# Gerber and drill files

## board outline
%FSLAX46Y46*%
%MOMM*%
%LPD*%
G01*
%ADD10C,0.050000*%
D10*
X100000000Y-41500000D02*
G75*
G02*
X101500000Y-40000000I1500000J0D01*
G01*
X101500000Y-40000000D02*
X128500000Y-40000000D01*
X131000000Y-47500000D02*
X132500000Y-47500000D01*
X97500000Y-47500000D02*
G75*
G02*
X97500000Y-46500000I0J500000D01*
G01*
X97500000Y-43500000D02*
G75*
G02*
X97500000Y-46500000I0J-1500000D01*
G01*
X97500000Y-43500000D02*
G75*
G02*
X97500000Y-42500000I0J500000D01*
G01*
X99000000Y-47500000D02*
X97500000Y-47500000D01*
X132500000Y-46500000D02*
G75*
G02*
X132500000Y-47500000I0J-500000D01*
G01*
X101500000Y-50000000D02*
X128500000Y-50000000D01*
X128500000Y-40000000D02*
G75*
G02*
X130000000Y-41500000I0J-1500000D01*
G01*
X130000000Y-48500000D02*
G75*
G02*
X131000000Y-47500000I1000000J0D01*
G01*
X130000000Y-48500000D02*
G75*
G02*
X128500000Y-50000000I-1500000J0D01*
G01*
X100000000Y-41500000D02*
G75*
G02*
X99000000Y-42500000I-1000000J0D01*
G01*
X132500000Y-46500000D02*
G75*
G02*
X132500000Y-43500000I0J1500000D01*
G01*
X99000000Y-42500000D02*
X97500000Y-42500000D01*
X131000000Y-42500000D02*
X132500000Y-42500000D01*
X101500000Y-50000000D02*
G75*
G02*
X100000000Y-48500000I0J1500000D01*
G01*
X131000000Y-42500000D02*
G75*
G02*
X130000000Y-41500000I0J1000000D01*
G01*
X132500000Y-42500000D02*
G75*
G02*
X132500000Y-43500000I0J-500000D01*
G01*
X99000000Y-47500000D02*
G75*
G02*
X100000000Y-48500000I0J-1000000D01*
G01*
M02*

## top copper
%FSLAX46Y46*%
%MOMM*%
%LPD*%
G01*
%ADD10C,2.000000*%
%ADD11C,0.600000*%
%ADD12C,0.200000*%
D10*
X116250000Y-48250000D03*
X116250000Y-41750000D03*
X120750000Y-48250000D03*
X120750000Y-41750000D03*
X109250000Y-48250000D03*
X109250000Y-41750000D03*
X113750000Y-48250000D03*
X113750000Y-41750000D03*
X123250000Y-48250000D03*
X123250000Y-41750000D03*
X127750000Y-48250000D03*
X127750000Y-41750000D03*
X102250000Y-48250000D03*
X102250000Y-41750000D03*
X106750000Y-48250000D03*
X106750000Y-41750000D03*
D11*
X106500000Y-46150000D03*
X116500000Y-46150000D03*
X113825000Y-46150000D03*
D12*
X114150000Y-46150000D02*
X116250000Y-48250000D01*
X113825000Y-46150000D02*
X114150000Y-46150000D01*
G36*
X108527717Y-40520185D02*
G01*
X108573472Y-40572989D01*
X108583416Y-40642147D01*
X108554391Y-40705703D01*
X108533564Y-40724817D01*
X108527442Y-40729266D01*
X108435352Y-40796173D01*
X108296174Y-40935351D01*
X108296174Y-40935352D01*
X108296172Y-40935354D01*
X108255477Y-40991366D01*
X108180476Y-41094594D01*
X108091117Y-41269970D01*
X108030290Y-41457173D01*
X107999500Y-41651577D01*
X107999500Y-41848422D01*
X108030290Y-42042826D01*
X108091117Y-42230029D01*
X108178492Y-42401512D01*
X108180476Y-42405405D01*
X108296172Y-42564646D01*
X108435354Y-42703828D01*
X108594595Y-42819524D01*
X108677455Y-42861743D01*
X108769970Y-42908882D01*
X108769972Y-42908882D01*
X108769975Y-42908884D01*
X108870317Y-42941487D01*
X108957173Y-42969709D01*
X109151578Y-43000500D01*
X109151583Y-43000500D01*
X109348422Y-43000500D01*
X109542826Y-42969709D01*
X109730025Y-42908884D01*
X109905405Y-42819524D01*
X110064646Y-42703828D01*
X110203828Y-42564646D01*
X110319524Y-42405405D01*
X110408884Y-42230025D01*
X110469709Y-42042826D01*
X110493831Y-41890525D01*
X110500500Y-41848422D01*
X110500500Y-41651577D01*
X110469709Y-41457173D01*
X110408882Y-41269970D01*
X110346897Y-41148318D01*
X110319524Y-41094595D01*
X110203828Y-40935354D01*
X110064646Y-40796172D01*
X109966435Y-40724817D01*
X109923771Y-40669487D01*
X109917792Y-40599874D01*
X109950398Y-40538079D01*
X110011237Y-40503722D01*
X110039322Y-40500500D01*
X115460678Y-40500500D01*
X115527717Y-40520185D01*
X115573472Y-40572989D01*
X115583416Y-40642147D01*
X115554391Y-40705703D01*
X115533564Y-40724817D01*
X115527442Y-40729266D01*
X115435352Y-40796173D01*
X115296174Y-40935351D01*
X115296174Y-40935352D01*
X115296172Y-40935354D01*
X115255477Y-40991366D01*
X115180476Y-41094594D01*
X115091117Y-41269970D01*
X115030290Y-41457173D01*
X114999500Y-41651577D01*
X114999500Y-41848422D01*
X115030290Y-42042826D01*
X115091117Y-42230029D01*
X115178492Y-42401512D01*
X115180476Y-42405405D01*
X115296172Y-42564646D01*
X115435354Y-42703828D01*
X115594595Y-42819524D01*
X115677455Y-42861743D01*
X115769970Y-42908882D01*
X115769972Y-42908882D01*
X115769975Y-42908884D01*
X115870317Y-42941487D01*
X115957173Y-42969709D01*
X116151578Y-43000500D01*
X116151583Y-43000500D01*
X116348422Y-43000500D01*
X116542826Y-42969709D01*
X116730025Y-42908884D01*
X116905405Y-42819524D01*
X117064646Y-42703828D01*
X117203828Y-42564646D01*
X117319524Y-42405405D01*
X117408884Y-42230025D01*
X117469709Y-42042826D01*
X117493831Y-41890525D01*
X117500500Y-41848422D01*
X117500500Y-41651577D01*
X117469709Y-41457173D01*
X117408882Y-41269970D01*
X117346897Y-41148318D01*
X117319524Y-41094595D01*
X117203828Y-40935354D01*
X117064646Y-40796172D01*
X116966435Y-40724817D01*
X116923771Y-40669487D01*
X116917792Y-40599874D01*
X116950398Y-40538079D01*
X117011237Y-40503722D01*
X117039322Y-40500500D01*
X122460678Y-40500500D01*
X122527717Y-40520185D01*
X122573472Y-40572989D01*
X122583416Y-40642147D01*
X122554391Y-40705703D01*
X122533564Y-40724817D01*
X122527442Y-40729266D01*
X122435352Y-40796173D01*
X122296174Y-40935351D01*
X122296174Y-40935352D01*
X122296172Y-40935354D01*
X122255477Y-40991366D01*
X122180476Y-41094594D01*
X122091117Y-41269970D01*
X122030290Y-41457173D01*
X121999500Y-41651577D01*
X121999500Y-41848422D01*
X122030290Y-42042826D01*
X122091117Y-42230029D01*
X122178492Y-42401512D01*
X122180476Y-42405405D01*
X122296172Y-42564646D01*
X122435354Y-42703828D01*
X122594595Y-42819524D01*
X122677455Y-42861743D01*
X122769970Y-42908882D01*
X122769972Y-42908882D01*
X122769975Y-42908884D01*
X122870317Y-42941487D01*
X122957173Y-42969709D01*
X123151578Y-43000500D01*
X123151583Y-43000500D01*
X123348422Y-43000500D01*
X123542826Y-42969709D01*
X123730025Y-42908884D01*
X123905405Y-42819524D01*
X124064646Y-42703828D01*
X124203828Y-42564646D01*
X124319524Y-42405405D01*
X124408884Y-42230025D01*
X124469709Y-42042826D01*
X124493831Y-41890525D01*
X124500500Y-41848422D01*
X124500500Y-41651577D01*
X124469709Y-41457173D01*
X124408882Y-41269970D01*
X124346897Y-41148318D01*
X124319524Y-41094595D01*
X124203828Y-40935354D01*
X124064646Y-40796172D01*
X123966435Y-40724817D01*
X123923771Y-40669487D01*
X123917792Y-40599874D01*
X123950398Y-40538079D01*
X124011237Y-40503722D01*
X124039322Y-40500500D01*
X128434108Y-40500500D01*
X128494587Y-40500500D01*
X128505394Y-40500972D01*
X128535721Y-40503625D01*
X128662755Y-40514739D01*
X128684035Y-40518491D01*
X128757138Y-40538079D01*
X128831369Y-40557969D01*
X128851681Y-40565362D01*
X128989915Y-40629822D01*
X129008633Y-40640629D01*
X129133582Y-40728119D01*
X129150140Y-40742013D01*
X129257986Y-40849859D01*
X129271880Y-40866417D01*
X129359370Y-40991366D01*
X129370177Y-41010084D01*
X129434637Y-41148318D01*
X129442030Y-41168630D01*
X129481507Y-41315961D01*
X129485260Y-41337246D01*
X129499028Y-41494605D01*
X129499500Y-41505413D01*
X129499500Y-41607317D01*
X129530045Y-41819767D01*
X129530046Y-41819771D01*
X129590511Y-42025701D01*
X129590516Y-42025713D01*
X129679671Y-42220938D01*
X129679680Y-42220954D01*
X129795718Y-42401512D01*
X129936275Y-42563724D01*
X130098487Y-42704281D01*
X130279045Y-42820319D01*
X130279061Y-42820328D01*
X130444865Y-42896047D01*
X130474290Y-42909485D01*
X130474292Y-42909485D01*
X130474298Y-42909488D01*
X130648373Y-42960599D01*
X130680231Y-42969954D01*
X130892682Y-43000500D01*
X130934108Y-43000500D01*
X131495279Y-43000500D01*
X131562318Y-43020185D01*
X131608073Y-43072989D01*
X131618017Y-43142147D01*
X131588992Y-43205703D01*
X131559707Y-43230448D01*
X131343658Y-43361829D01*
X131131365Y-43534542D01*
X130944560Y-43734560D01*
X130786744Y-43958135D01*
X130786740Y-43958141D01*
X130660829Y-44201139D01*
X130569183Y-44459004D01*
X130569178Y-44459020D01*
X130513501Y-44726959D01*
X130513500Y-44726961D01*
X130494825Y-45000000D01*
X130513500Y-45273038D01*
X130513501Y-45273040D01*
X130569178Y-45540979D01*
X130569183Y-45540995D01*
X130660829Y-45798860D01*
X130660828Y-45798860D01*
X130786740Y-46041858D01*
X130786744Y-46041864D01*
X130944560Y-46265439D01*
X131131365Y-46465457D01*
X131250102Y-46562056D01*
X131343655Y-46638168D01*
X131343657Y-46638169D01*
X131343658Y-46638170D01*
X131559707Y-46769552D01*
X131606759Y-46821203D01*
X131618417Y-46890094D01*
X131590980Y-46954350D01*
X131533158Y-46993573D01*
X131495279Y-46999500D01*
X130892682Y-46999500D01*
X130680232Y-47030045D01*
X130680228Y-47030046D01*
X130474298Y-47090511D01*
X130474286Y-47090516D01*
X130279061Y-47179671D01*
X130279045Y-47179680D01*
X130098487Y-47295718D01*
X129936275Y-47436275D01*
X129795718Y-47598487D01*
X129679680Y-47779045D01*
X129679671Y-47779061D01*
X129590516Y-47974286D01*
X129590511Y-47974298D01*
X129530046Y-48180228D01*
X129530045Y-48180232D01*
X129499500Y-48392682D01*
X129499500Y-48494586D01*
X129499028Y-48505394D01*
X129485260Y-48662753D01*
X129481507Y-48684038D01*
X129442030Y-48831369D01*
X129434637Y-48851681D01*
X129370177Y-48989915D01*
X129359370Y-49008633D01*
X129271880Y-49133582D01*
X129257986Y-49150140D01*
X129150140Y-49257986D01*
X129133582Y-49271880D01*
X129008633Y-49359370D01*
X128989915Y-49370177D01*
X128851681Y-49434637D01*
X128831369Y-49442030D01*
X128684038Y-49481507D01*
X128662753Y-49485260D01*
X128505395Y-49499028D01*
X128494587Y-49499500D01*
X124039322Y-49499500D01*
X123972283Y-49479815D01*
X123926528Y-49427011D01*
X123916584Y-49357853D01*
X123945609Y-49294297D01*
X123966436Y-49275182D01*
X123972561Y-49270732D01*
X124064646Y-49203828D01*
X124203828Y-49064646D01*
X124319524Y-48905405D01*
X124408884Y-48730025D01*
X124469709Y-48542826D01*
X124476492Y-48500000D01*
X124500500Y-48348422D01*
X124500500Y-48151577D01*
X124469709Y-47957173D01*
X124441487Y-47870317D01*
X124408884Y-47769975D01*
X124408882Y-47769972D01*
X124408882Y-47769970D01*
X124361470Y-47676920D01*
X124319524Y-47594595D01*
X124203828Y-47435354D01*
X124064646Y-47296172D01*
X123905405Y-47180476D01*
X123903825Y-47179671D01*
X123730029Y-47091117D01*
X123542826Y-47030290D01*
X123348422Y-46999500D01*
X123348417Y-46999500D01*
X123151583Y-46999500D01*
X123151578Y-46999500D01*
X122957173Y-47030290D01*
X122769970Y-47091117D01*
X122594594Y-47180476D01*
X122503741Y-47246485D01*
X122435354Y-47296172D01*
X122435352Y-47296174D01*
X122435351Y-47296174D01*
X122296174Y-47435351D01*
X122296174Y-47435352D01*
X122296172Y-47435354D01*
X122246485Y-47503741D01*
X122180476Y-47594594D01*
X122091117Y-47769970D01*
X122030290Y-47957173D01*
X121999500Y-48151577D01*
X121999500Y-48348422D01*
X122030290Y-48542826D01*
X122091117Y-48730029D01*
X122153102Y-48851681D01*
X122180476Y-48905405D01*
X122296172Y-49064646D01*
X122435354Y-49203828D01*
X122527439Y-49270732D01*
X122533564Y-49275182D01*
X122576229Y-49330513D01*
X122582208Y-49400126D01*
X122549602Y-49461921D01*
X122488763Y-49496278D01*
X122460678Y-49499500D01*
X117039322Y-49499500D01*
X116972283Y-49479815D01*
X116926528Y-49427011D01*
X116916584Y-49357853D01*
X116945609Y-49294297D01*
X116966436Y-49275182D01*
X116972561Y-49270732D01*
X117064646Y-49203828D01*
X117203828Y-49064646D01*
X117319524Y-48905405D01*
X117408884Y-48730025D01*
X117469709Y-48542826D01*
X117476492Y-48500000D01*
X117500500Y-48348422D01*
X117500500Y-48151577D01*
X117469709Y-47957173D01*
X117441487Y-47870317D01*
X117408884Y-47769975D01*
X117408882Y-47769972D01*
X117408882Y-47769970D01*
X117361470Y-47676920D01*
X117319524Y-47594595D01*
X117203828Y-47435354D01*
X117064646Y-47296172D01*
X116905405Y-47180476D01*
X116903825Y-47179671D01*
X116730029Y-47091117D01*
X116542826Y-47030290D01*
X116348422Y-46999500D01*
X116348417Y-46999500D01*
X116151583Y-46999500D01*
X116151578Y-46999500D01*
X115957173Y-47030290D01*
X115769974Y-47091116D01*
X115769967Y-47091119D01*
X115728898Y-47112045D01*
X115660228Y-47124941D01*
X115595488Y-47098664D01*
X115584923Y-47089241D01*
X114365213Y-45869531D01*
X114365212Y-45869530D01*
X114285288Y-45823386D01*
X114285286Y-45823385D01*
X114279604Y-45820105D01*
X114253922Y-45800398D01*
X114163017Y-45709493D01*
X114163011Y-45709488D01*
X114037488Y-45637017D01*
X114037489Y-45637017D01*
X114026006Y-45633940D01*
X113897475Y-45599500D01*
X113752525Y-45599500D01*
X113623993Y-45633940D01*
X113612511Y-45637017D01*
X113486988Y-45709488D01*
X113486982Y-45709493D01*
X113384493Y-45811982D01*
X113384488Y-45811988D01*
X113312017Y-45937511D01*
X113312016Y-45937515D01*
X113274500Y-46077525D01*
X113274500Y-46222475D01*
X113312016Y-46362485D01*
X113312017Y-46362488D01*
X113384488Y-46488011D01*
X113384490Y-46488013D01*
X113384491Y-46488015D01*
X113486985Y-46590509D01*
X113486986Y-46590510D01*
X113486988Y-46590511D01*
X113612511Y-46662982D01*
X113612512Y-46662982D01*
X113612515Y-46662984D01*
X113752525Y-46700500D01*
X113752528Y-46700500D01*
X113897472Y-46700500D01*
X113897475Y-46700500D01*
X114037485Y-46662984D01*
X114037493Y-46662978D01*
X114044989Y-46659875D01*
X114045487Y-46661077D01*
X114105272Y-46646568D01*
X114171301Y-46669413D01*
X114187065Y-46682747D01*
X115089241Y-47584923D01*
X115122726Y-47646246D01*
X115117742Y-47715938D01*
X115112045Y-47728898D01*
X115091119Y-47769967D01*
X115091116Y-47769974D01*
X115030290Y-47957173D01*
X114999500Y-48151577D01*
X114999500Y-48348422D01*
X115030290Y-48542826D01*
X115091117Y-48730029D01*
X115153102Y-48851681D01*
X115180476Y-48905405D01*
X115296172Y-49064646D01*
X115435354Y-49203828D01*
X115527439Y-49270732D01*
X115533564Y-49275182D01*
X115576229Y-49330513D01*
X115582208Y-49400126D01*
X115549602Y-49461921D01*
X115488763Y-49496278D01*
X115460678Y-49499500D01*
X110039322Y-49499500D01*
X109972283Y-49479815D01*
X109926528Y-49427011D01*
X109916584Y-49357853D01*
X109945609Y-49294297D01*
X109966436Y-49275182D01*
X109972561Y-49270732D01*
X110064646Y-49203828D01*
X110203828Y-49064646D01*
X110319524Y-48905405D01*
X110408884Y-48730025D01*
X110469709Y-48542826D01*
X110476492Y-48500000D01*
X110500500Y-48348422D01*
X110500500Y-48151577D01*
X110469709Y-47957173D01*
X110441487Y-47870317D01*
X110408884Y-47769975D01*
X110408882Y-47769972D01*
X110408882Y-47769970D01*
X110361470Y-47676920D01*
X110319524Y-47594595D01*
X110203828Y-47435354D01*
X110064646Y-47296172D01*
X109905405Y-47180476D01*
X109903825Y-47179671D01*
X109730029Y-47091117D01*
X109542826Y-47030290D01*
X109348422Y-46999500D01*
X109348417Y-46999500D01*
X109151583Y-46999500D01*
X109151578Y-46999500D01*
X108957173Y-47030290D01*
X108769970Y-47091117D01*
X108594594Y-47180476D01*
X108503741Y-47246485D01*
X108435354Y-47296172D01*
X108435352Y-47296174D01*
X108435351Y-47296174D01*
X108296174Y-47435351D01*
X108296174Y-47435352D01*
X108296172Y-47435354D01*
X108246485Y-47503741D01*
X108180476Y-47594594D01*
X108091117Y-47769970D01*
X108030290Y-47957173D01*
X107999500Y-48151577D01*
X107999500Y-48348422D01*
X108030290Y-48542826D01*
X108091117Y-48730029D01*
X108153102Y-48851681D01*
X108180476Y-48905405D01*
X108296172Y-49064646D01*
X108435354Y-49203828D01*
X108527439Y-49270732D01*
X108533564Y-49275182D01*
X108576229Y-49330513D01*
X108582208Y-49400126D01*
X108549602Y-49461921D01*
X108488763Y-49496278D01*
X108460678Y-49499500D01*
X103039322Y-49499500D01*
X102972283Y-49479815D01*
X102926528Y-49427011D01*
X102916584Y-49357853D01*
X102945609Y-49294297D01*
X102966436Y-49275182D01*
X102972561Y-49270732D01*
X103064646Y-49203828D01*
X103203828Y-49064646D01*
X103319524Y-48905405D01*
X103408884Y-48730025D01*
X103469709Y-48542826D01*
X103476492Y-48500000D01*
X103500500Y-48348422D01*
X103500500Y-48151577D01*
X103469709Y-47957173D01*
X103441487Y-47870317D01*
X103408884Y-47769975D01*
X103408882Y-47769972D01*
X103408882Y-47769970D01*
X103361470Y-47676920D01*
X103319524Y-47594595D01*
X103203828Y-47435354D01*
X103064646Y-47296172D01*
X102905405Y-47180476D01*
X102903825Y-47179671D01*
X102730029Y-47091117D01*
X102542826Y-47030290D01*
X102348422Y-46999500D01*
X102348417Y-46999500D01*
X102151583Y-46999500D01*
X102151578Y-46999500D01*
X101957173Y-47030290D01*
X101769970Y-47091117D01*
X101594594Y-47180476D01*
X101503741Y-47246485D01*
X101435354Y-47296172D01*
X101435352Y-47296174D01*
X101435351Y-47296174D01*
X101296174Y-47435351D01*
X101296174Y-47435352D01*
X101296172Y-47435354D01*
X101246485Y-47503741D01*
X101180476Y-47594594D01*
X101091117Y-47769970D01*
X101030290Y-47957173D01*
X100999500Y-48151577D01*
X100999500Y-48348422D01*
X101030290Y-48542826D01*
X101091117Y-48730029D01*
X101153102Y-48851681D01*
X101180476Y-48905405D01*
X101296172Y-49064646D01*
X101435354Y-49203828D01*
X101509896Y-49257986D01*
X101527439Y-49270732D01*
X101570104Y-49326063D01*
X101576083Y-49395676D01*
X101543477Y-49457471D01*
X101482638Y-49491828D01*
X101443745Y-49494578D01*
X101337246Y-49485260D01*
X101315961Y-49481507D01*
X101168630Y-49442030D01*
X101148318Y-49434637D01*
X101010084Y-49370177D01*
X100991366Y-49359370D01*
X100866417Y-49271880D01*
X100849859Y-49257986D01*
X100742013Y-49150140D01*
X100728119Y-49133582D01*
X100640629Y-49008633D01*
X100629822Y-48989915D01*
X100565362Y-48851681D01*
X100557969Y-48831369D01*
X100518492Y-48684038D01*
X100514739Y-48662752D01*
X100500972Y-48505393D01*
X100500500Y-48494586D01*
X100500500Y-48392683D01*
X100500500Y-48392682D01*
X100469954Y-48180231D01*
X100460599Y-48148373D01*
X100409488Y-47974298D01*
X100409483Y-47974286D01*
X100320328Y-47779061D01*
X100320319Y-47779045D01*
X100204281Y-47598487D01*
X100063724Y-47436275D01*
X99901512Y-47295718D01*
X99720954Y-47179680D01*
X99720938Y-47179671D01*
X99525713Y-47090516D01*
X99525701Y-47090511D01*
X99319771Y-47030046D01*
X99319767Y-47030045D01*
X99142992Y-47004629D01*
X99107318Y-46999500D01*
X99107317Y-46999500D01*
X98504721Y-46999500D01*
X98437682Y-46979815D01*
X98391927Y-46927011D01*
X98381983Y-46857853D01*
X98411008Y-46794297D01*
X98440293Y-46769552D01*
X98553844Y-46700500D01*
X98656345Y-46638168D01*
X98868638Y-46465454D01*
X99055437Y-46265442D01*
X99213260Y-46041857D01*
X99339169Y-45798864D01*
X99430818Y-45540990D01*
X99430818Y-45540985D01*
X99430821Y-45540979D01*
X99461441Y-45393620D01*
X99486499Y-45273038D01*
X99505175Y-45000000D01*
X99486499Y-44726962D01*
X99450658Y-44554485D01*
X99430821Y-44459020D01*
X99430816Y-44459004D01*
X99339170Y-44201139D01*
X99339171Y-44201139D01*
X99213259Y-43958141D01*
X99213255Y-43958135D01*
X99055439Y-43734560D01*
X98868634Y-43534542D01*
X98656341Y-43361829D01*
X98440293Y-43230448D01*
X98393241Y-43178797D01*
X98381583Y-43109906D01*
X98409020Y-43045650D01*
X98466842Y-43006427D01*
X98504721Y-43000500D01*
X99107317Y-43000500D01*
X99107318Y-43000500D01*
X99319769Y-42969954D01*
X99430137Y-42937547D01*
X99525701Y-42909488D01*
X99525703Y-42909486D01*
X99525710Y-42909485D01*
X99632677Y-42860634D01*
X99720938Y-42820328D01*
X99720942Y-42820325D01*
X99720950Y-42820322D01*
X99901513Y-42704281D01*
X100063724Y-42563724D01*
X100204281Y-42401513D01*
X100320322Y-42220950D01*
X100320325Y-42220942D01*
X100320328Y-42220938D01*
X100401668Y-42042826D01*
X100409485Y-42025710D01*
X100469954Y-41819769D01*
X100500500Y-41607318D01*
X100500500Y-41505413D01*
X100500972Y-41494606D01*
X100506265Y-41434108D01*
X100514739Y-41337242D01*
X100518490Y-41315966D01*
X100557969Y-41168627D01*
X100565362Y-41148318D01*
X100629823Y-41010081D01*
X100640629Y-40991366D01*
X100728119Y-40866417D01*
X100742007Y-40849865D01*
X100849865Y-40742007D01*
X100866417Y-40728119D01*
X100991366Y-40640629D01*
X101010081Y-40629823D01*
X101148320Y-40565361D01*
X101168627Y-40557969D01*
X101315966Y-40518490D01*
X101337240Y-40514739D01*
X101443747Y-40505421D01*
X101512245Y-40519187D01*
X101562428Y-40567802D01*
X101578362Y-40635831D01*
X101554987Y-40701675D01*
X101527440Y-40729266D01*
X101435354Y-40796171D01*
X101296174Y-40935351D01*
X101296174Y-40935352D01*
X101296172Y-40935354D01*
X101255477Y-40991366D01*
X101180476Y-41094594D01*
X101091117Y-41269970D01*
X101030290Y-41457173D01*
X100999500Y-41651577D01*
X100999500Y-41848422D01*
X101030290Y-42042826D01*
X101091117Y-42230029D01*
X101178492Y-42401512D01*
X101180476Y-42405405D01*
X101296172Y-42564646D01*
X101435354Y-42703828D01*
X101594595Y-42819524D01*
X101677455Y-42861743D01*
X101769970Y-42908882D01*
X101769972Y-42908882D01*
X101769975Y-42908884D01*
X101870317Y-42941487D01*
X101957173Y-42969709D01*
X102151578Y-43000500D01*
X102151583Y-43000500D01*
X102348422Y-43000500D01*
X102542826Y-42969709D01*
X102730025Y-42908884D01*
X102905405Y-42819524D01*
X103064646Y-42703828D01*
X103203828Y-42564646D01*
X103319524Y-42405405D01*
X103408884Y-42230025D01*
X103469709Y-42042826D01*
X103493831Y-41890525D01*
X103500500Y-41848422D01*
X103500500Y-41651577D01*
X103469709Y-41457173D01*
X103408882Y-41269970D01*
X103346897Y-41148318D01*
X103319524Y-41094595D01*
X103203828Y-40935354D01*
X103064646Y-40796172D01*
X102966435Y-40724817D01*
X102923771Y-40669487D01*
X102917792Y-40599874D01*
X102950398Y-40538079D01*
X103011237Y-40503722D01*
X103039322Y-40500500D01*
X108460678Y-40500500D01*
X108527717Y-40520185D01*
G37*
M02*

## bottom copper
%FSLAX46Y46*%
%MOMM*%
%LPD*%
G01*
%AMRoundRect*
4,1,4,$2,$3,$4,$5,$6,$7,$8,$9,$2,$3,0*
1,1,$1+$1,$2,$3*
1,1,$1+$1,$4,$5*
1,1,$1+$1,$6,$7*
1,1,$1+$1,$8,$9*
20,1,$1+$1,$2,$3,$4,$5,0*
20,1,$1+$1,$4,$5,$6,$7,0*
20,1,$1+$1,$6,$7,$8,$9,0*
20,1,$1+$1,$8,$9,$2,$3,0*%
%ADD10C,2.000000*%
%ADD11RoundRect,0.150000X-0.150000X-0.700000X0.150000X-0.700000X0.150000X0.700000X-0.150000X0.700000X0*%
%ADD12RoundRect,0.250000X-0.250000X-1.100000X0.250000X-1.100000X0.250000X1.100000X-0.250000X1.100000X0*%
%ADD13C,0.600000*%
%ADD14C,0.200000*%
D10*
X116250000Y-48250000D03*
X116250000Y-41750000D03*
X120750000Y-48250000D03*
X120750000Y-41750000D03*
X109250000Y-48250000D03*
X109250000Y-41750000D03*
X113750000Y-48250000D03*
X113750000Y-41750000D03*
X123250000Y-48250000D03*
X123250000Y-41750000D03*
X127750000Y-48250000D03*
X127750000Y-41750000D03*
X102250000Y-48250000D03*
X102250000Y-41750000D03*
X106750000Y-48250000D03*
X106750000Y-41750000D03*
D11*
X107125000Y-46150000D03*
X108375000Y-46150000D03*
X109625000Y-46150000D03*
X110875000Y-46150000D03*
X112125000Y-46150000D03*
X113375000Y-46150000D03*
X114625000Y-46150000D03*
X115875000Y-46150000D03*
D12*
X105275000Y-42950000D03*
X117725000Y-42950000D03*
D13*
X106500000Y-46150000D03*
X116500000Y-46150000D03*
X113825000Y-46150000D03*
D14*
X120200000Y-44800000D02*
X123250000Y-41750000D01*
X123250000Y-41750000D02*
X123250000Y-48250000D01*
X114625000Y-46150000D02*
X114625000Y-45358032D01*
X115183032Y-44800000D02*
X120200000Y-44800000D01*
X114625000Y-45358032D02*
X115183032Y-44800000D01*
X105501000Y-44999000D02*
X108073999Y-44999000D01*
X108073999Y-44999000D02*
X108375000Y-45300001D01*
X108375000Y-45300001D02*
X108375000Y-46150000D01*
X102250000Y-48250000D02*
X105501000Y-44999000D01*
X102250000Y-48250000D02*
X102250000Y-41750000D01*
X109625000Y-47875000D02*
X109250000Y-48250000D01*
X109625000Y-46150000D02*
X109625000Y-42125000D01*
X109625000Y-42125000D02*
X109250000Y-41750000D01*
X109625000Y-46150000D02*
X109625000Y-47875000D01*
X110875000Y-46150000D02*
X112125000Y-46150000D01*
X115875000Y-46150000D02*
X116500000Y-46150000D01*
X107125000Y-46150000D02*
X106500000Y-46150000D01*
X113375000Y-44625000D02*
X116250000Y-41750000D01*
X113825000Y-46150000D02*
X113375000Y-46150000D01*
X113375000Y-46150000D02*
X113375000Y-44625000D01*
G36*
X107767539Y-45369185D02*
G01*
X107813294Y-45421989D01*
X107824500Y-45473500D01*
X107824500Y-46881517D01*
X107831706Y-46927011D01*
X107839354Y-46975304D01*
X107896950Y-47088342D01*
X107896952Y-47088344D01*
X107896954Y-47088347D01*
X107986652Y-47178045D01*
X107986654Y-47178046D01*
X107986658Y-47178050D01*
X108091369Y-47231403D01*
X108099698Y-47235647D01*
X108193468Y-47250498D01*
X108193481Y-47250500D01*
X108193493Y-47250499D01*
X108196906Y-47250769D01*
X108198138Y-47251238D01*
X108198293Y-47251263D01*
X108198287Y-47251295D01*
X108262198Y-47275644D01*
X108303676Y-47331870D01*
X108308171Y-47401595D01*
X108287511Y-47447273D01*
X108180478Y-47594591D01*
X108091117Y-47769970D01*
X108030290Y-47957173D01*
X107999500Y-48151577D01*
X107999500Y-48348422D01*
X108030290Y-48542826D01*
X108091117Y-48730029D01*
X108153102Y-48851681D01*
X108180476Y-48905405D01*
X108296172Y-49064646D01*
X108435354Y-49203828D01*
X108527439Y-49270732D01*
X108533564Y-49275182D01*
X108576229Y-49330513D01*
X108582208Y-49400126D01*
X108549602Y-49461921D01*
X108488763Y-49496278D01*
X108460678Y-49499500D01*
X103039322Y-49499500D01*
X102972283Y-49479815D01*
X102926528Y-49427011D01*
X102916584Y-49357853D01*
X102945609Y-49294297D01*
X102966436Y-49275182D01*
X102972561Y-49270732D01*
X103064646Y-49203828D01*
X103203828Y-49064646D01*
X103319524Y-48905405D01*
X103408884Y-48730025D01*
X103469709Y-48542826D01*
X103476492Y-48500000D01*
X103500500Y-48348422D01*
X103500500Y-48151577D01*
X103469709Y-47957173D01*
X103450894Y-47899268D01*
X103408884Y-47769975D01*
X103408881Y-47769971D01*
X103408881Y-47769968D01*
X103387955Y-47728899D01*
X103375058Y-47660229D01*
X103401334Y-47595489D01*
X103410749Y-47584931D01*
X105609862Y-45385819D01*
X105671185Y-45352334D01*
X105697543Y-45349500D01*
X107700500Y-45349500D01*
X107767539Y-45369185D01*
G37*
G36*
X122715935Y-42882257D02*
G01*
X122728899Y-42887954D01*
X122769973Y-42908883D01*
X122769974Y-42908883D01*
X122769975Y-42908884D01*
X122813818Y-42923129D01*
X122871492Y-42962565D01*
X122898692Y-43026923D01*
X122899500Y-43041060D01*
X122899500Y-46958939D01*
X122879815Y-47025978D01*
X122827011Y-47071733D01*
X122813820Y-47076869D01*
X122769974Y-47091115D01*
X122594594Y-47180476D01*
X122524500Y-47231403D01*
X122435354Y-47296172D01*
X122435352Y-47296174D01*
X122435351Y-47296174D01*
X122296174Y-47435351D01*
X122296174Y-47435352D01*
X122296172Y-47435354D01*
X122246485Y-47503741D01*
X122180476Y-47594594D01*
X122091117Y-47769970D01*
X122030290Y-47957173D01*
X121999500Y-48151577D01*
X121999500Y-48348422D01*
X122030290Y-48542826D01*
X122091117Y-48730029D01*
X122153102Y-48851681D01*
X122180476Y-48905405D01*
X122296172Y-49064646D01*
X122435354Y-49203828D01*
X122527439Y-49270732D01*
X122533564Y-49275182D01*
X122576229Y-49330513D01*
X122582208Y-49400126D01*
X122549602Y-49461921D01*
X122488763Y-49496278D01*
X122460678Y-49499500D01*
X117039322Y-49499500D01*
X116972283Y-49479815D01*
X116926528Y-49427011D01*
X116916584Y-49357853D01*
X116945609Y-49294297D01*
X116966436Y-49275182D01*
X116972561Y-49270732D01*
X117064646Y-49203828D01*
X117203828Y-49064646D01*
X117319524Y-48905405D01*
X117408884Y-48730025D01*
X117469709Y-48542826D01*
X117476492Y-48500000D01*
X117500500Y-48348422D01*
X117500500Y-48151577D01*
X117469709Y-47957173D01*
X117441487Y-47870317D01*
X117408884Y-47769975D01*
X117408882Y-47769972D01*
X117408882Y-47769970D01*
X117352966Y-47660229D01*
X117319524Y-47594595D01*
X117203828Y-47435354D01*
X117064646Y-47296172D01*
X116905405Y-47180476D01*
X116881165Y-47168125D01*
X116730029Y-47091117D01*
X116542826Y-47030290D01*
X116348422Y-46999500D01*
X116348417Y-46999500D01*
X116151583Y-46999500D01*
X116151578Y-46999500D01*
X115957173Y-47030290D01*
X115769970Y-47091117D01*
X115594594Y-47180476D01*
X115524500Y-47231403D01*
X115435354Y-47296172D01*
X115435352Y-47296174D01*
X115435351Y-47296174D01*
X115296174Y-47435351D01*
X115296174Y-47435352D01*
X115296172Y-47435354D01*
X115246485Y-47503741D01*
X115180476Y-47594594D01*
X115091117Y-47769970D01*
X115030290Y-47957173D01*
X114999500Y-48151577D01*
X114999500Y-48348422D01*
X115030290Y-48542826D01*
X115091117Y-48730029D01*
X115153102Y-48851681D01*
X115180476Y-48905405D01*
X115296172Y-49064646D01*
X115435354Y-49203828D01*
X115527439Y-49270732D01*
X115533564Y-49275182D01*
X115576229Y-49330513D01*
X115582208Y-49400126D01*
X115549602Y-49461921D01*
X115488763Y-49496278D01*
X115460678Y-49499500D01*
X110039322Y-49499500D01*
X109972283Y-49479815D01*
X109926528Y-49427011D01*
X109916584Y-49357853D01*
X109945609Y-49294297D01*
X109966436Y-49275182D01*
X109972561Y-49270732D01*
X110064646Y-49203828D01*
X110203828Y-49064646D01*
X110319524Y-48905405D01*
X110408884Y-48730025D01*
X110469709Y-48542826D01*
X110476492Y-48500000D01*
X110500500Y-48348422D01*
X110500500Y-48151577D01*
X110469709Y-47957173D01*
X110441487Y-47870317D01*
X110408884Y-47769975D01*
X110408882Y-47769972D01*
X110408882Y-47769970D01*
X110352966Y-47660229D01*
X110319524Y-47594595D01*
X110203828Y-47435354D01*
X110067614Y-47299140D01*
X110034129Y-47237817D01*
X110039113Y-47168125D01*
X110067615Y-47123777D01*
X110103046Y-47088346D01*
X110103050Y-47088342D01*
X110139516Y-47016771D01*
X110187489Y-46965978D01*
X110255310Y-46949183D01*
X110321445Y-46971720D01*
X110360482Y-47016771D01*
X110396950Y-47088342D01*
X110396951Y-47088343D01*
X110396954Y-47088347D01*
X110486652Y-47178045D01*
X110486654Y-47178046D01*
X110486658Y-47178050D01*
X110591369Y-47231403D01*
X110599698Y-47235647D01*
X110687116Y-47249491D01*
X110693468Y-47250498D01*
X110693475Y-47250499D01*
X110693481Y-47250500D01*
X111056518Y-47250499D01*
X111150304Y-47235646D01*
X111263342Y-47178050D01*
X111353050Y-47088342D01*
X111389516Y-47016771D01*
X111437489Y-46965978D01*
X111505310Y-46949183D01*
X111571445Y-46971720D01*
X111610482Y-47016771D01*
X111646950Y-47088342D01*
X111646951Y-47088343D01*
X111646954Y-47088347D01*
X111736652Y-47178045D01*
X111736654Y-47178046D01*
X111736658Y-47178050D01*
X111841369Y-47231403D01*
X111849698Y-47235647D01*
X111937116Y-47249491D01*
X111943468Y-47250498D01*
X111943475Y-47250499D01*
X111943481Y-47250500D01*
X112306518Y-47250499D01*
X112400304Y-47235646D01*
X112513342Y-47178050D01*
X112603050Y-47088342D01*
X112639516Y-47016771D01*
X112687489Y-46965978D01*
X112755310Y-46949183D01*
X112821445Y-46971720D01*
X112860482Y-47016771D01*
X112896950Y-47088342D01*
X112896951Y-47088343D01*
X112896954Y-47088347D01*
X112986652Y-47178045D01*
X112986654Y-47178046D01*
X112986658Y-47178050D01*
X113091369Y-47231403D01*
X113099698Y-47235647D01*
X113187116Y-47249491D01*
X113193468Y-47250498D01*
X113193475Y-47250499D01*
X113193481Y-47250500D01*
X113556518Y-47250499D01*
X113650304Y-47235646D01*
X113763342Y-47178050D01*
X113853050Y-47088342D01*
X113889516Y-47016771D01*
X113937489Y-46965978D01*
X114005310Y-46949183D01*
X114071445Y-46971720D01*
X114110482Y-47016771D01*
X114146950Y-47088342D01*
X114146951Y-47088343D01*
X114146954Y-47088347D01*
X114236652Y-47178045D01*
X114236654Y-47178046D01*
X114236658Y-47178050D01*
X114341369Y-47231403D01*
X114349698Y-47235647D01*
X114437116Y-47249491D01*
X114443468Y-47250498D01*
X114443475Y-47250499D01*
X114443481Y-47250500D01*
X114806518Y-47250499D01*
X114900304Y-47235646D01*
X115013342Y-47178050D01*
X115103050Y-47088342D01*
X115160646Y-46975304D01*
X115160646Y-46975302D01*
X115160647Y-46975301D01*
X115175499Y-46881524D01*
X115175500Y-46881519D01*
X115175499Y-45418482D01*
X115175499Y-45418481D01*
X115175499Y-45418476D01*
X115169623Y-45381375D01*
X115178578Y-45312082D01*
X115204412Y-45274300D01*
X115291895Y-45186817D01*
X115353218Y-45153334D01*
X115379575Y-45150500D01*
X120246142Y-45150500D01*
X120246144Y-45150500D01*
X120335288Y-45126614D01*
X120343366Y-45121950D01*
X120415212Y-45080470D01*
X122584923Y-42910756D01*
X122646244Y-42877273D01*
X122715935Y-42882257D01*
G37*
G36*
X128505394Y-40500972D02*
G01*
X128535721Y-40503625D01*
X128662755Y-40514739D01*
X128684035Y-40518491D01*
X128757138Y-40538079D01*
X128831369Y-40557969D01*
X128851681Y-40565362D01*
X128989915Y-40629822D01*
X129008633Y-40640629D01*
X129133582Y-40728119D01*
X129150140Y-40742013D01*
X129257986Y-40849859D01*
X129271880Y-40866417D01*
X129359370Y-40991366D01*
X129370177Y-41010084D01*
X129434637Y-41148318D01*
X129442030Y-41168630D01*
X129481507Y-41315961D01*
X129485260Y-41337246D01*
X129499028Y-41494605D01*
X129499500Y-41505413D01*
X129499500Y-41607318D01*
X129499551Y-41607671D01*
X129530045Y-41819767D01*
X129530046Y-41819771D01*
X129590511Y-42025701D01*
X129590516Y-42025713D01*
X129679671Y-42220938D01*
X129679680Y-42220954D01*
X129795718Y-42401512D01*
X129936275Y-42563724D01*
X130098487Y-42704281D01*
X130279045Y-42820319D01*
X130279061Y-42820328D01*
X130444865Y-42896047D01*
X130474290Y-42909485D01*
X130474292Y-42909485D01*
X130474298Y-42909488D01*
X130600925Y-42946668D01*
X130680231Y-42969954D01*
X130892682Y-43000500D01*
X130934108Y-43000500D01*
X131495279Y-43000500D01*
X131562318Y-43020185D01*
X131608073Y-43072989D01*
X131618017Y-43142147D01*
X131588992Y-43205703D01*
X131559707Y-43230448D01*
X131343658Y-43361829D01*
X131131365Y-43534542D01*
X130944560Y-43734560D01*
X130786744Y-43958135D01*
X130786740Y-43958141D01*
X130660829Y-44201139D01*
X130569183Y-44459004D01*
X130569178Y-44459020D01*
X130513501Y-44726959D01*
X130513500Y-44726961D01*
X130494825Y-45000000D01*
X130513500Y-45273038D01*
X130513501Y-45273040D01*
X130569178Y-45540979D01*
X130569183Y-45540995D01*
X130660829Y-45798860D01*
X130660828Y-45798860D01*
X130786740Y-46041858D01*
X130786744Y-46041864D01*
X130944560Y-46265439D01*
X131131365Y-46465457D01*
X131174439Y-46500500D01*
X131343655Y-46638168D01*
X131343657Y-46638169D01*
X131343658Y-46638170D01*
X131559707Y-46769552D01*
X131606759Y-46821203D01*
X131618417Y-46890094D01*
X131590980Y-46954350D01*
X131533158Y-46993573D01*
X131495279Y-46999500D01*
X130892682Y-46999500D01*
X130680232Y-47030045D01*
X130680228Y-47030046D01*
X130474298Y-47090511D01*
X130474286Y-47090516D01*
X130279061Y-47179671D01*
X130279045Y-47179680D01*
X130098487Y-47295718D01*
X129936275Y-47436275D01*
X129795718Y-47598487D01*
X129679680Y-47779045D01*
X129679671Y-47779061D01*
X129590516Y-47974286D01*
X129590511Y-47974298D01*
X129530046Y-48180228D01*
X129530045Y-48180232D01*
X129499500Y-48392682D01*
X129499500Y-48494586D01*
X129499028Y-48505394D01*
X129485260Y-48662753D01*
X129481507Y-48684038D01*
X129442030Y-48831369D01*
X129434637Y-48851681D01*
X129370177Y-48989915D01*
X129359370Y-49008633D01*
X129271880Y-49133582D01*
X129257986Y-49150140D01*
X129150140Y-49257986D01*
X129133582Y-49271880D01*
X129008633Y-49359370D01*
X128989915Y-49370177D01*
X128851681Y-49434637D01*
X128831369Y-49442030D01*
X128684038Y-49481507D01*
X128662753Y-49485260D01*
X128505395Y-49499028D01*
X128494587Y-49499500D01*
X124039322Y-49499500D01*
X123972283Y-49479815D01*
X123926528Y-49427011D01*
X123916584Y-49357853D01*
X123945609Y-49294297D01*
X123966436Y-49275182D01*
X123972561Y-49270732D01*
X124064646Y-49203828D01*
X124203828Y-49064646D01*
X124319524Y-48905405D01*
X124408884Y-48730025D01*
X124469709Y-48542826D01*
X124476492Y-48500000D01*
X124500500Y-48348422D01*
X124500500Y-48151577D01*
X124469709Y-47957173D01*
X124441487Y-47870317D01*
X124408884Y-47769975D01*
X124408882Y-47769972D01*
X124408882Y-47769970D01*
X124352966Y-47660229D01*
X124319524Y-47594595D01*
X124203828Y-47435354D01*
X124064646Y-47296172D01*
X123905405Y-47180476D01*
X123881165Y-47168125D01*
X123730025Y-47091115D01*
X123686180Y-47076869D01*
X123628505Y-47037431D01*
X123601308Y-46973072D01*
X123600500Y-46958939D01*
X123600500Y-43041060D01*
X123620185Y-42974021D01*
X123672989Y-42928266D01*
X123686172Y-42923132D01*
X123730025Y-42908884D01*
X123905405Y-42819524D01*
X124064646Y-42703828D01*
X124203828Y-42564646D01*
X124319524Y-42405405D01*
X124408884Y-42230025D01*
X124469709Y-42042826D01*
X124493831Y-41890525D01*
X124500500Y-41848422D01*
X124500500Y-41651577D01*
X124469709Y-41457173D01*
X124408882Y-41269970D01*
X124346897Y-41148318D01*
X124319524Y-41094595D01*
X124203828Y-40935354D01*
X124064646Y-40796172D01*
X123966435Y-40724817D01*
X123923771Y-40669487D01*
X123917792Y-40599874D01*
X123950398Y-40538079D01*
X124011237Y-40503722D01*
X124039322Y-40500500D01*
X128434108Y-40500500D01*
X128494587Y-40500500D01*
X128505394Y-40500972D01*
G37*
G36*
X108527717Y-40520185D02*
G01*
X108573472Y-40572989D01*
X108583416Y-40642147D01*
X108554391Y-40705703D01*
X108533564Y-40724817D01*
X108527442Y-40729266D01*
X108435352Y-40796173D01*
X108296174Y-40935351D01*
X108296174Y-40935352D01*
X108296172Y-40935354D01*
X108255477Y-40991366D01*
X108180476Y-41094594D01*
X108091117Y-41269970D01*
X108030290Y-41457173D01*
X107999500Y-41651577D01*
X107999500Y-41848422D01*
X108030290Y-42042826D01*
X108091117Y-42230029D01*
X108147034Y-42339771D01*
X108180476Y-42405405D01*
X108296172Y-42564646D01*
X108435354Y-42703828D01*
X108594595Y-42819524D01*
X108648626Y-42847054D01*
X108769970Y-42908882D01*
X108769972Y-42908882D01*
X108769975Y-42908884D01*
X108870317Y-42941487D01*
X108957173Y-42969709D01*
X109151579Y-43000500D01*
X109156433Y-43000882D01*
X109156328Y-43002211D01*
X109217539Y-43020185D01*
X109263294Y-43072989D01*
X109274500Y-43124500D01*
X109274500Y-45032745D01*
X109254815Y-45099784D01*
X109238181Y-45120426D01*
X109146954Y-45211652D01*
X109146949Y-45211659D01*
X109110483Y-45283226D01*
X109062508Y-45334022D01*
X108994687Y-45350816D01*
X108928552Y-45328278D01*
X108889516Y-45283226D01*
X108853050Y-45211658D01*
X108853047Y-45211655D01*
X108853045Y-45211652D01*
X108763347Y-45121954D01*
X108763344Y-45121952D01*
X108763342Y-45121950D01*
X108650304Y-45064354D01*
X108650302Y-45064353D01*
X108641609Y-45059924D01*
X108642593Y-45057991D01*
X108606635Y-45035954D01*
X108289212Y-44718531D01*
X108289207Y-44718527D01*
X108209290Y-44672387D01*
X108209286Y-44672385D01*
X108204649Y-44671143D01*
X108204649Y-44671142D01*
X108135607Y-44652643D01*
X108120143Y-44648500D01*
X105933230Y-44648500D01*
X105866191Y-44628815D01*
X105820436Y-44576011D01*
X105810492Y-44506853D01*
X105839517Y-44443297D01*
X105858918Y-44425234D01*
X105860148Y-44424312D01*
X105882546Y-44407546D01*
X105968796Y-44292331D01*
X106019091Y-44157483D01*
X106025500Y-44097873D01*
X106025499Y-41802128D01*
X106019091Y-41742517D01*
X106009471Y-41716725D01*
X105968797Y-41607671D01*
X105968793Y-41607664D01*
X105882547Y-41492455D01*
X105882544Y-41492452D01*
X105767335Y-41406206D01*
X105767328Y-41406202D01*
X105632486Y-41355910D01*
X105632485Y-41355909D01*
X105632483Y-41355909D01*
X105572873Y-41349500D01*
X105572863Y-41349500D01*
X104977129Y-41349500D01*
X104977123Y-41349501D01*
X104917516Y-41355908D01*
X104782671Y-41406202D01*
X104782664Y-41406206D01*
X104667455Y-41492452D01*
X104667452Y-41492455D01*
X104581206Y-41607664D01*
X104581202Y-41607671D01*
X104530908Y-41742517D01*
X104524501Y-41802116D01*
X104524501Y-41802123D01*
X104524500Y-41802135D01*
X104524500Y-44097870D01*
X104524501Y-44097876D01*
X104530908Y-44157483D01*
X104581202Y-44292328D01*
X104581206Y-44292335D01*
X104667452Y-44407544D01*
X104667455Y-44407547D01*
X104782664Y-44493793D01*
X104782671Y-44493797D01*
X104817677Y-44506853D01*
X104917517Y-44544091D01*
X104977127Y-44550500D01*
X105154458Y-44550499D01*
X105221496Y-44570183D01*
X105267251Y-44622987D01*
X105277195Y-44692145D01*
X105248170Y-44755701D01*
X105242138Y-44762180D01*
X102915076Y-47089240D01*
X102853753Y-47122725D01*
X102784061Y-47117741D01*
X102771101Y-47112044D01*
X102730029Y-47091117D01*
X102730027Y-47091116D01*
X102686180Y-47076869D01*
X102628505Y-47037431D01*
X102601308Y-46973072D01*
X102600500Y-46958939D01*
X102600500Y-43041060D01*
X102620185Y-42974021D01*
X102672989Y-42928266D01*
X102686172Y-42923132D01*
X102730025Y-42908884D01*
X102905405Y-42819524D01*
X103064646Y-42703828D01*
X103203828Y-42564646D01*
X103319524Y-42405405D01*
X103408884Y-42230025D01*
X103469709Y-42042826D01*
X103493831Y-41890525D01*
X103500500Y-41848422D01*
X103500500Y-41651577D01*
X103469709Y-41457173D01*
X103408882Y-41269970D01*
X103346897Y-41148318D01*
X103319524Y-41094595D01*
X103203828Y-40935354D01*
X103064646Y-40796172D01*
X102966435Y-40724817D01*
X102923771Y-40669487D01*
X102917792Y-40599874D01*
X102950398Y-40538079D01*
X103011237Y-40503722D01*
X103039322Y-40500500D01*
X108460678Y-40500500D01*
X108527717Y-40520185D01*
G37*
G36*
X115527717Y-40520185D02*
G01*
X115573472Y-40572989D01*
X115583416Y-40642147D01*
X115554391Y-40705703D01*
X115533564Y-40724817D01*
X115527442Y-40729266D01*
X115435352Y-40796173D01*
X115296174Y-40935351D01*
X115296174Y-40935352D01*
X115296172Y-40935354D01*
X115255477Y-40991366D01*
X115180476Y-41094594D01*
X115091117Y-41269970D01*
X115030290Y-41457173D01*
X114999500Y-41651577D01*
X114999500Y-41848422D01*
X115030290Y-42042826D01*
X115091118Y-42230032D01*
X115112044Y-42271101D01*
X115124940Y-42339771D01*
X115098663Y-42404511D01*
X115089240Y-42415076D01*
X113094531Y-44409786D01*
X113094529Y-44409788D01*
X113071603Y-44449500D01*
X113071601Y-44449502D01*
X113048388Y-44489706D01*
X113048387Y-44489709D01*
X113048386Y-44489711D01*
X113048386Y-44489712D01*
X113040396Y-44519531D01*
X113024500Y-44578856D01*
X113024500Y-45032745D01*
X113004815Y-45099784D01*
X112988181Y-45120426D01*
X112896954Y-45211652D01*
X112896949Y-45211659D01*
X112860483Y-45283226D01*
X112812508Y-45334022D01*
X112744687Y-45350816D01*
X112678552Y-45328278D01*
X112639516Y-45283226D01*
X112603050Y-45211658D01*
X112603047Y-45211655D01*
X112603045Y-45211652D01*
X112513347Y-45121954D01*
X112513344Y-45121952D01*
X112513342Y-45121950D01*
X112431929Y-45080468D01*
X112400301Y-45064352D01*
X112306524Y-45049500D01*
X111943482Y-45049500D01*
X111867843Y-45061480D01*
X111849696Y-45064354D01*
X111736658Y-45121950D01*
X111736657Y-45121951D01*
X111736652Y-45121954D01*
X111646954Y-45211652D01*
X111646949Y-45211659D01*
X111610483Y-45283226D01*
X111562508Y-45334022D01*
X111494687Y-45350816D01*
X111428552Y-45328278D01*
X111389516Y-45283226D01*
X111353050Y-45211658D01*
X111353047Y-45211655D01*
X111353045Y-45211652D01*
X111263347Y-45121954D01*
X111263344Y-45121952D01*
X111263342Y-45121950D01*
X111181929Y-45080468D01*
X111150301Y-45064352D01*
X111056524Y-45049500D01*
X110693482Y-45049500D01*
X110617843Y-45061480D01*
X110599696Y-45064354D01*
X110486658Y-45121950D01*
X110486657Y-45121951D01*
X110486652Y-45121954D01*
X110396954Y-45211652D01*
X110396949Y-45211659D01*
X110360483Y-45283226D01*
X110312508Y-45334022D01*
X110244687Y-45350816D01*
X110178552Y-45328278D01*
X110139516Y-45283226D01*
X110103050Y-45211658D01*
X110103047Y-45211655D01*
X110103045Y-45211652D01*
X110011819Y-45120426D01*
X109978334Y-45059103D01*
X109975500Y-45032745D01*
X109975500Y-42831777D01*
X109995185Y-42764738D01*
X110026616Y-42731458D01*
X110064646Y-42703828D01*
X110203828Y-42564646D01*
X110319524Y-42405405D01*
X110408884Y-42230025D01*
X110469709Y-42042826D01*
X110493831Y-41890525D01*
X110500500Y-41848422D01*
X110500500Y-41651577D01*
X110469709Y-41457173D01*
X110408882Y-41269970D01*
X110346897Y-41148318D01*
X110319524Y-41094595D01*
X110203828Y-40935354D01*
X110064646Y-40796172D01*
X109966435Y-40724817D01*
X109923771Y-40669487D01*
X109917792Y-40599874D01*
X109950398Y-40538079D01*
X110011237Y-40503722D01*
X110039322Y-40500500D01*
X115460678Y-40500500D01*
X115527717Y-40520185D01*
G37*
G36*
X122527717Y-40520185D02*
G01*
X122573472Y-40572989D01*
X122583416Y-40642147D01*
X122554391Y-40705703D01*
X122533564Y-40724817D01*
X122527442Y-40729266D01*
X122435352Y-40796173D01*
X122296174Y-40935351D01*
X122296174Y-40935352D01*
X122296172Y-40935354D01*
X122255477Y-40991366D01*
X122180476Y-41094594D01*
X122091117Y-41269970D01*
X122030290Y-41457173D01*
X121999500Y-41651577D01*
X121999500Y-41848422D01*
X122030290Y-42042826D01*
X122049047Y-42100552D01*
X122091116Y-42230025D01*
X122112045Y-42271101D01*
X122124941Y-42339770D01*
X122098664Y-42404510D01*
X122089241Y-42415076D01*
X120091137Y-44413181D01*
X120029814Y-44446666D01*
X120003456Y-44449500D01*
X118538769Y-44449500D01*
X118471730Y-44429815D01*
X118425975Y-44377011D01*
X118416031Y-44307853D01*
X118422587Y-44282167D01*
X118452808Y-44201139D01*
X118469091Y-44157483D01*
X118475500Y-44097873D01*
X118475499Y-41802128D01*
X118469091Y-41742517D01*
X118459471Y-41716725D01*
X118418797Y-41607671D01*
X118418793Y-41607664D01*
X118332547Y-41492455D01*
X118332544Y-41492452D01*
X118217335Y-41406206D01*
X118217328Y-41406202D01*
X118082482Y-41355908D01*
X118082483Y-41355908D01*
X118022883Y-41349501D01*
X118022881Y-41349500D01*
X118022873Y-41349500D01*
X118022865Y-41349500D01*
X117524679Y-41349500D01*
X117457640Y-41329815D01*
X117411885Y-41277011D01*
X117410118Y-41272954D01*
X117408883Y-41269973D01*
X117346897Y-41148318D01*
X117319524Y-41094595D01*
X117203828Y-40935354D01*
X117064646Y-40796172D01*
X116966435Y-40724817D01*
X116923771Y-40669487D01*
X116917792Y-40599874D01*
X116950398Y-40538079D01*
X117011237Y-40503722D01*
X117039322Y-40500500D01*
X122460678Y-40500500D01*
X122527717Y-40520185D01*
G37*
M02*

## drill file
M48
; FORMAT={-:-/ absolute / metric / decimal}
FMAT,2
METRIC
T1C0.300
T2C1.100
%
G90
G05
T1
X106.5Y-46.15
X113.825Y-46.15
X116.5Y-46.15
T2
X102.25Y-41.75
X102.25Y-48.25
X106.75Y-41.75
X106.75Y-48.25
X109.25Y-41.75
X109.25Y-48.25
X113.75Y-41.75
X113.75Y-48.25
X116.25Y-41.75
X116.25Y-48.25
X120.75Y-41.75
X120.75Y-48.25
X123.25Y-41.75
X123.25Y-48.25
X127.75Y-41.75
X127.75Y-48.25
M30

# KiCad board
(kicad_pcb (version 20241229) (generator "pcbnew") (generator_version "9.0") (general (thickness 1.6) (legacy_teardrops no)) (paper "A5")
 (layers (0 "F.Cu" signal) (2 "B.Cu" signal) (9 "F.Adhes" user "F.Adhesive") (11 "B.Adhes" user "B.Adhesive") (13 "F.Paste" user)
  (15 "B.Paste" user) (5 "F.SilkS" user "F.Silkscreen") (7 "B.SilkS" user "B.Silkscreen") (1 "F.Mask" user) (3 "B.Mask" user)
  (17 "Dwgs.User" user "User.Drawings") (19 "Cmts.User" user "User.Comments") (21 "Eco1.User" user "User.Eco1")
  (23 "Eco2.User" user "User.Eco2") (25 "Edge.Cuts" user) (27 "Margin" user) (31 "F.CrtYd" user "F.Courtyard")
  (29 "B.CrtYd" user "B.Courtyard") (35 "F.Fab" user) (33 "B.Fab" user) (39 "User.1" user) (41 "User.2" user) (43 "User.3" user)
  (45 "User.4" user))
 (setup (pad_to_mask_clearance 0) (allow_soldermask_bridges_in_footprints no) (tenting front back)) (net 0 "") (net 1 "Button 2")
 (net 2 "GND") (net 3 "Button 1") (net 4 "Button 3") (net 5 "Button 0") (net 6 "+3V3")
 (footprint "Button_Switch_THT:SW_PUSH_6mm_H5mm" (layer "F.Cu") (at 116.25 48.25 90)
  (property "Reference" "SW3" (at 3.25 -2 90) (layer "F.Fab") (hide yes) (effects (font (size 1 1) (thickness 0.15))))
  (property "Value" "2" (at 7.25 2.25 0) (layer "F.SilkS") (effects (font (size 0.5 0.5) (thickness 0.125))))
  (pad "1" thru_hole circle (at 0 0 180) (size 2 2) (drill 1.1) (layers "*.Cu" "*.Mask") (remove_unused_layers no) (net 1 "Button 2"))
  (pad "1" thru_hole circle (at 6.5 0 180) (size 2 2) (drill 1.1) (layers "*.Cu" "*.Mask") (remove_unused_layers no) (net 1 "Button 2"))
  (pad "2" thru_hole circle (at 0 4.5 180) (size 2 2) (drill 1.1) (layers "*.Cu" "*.Mask") (remove_unused_layers no) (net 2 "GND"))
  (pad "2" thru_hole circle (at 6.5 4.5 180) (size 2 2) (drill 1.1) (layers "*.Cu" "*.Mask") (remove_unused_layers no) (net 2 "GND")))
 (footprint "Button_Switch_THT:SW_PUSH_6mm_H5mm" (layer "F.Cu") (at 109.25 48.25 90)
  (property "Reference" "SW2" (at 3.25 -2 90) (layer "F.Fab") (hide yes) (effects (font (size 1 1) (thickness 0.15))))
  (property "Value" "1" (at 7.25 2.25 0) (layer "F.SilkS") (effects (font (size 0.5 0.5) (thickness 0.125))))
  (pad "1" thru_hole circle (at 0 0 180) (size 2 2) (drill 1.1) (layers "*.Cu" "*.Mask") (remove_unused_layers no) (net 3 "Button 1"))
  (pad "1" thru_hole circle (at 6.5 0 180) (size 2 2) (drill 1.1) (layers "*.Cu" "*.Mask") (remove_unused_layers no) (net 3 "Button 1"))
  (pad "2" thru_hole circle (at 0 4.5 180) (size 2 2) (drill 1.1) (layers "*.Cu" "*.Mask") (remove_unused_layers no) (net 2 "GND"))
  (pad "2" thru_hole circle (at 6.5 4.5 180) (size 2 2) (drill 1.1) (layers "*.Cu" "*.Mask") (remove_unused_layers no) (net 2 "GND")))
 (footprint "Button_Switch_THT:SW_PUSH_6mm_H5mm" (layer "F.Cu") (at 123.25 48.25 90)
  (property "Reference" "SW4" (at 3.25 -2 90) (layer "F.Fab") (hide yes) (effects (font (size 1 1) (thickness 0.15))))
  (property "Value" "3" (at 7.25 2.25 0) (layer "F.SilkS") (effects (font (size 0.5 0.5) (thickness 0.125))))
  (pad "1" thru_hole circle (at 0 0 180) (size 2 2) (drill 1.1) (layers "*.Cu" "*.Mask") (remove_unused_layers no) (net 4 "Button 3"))
  (pad "1" thru_hole circle (at 6.5 0 180) (size 2 2) (drill 1.1) (layers "*.Cu" "*.Mask") (remove_unused_layers no) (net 4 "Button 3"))
  (pad "2" thru_hole circle (at 0 4.5 180) (size 2 2) (drill 1.1) (layers "*.Cu" "*.Mask") (remove_unused_layers no) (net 2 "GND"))
  (pad "2" thru_hole circle (at 6.5 4.5 180) (size 2 2) (drill 1.1) (layers "*.Cu" "*.Mask") (remove_unused_layers no) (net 2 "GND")))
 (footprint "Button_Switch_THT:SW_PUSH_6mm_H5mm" (layer "F.Cu") (at 102.25 48.25 90)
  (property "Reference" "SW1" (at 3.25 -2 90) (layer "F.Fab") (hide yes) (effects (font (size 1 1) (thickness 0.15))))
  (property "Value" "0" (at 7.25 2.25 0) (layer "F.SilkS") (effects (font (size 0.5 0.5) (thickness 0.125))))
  (pad "1" thru_hole circle (at 0 0 180) (size 2 2) (drill 1.1) (layers "*.Cu" "*.Mask") (remove_unused_layers no) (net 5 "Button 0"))
  (pad "1" thru_hole circle (at 6.5 0 180) (size 2 2) (drill 1.1) (layers "*.Cu" "*.Mask") (remove_unused_layers no) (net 5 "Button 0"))
  (pad "2" thru_hole circle (at 0 4.5 180) (size 2 2) (drill 1.1) (layers "*.Cu" "*.Mask") (remove_unused_layers no) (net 2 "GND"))
  (pad "2" thru_hole circle (at 6.5 4.5 180) (size 2 2) (drill 1.1) (layers "*.Cu" "*.Mask") (remove_unused_layers no) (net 2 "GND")))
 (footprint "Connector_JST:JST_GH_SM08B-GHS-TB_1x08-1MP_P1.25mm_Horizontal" (layer "B.Cu") (at 111.5 44.3)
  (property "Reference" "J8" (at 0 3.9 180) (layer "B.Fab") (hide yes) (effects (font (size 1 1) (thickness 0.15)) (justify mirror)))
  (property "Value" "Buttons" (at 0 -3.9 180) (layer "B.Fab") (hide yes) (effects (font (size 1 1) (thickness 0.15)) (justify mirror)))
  (pad "1" smd roundrect (at -4.375 1.85) (size 0.6 1.7) (layers "B.Cu" "B.Mask" "B.Paste") (roundrect_rratio 0.25) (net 2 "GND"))
  (pad "2" smd roundrect (at -3.125 1.85) (size 0.6 1.7) (layers "B.Cu" "B.Mask" "B.Paste") (roundrect_rratio 0.25) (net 5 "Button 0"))
  (pad "3" smd roundrect (at -1.875 1.85) (size 0.6 1.7) (layers "B.Cu" "B.Mask" "B.Paste") (roundrect_rratio 0.25) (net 3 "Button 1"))
  (pad "4" smd roundrect (at -0.625 1.85) (size 0.6 1.7) (layers "B.Cu" "B.Mask" "B.Paste") (roundrect_rratio 0.25) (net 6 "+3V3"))
  (pad "5" smd roundrect (at 0.625 1.85) (size 0.6 1.7) (layers "B.Cu" "B.Mask" "B.Paste") (roundrect_rratio 0.25) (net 6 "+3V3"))
  (pad "6" smd roundrect (at 1.875 1.85) (size 0.6 1.7) (layers "B.Cu" "B.Mask" "B.Paste") (roundrect_rratio 0.25) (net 1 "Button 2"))
  (pad "7" smd roundrect (at 3.125 1.85) (size 0.6 1.7) (layers "B.Cu" "B.Mask" "B.Paste") (roundrect_rratio 0.25) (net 4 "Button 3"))
  (pad "8" smd roundrect (at 4.375 1.85) (size 0.6 1.7) (layers "B.Cu" "B.Mask" "B.Paste") (roundrect_rratio 0.25) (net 2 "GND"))
  (pad "MP" smd roundrect (at -6.225 -1.35) (size 1 2.7) (layers "B.Cu" "B.Mask" "B.Paste") (roundrect_rratio 0.25))
  (pad "MP" smd roundrect (at 6.225 -1.35) (size 1 2.7) (layers "B.Cu" "B.Mask" "B.Paste") (roundrect_rratio 0.25)))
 (gr_arc (start 100 41.5) (mid 100.43934 40.43934) (end 101.5 40) (stroke (width 0.05) (type default)) (layer "Edge.Cuts"))
 (gr_line (start 101.5 40) (end 128.5 40) (stroke (width 0.05) (type default)) (layer "Edge.Cuts"))
 (gr_line (start 131 47.5) (end 132.5 47.5) (stroke (width 0.05) (type default)) (layer "Edge.Cuts"))
 (gr_arc (start 97.5 47.5) (mid 97 47) (end 97.5 46.5) (stroke (width 0.05) (type default)) (layer "Edge.Cuts"))
 (gr_arc (start 97.5 43.5) (mid 99 45) (end 97.5 46.5) (stroke (width 0.05) (type default)) (layer "Edge.Cuts"))
 (gr_arc (start 97.5 43.5) (mid 97 43) (end 97.5 42.5) (stroke (width 0.05) (type default)) (layer "Edge.Cuts"))
 (gr_line (start 99 47.5) (end 97.5 47.5) (stroke (width 0.05) (type default)) (layer "Edge.Cuts"))
 (gr_arc (start 132.5 46.5) (mid 133 47) (end 132.5 47.5) (stroke (width 0.05) (type default)) (layer "Edge.Cuts"))
 (gr_line (start 101.5 50) (end 128.5 50) (stroke (width 0.05) (type default)) (layer "Edge.Cuts"))
 (gr_arc (start 128.5 40) (mid 129.56066 40.43934) (end 130 41.5) (stroke (width 0.05) (type default)) (layer "Edge.Cuts"))
 (gr_arc (start 130 48.5) (mid 130.292893 47.792893) (end 131 47.5) (stroke (width 0.05) (type default)) (layer "Edge.Cuts"))
 (gr_arc (start 130 48.5) (mid 129.56066 49.56066) (end 128.5 50) (stroke (width 0.05) (type default)) (layer "Edge.Cuts"))
 (gr_arc (start 100 41.5) (mid 99.707107 42.207107) (end 99 42.5) (stroke (width 0.05) (type default)) (layer "Edge.Cuts"))
 (gr_arc (start 132.5 46.5) (mid 131 45) (end 132.5 43.5) (stroke (width 0.05) (type default)) (layer "Edge.Cuts"))
 (gr_line (start 99 42.5) (end 97.5 42.5) (stroke (width 0.05) (type default)) (layer "Edge.Cuts"))
 (gr_line (start 131 42.5) (end 132.5 42.5) (stroke (width 0.05) (type default)) (layer "Edge.Cuts"))
 (gr_arc (start 101.5 50) (mid 100.43934 49.56066) (end 100 48.5) (stroke (width 0.05) (type default)) (layer "Edge.Cuts"))
 (gr_arc (start 131 42.5) (mid 130.292893 42.207107) (end 130 41.5) (stroke (width 0.05) (type default)) (layer "Edge.Cuts"))
 (gr_arc (start 132.5 42.5) (mid 133 43) (end 132.5 43.5) (stroke (width 0.05) (type default)) (layer "Edge.Cuts"))
 (gr_arc (start 99 47.5) (mid 99.707107 47.792893) (end 100 48.5) (stroke (width 0.05) (type default)) (layer "Edge.Cuts"))
 (segment (start 120.2 44.8) (end 123.25 41.75) (width 0.2) (layer "B.Cu") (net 4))
 (segment (start 123.25 41.75) (end 123.25 48.25) (width 0.2) (layer "B.Cu") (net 4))
 (segment (start 114.625 46.15) (end 114.625 45.358032) (width 0.2) (layer "B.Cu") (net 4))
 (segment (start 115.183032 44.8) (end 120.2 44.8) (width 0.2) (layer "B.Cu") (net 4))
 (segment (start 114.625 45.358032) (end 115.183032 44.8) (width 0.2) (layer "B.Cu") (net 4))
 (segment (start 105.501 44.999) (end 108.073999 44.999) (width 0.2) (layer "B.Cu") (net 5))
 (segment (start 108.073999 44.999) (end 108.375 45.300001) (width 0.2) (layer "B.Cu") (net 5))
 (segment (start 108.375 45.300001) (end 108.375 46.15) (width 0.2) (layer "B.Cu") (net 5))
 (segment (start 102.25 48.25) (end 105.501 44.999) (width 0.2) (layer "B.Cu") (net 5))
 (segment (start 102.25 48.25) (end 102.25 41.75) (width 0.2) (layer "B.Cu") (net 5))
 (segment (start 109.625 47.875) (end 109.25 48.25) (width 0.2) (layer "B.Cu") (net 3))
 (segment (start 109.625 46.15) (end 109.625 42.125) (width 0.2) (layer "B.Cu") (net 3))
 (segment (start 109.625 42.125) (end 109.25 41.75) (width 0.2) (layer "B.Cu") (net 3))
 (segment (start 109.625 46.15) (end 109.625 47.875) (width 0.2) (layer "B.Cu") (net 3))
 (segment (start 110.875 46.15) (end 112.125 46.15) (width 0.2) (layer "B.Cu") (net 6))
 (via (at 106.5 46.15) (size 0.6) (drill 0.3) (layers "F.Cu" "B.Cu") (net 2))
 (via (at 116.5 46.15) (size 0.6) (drill 0.3) (layers "F.Cu" "B.Cu") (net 2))
 (segment (start 115.875 46.15) (end 116.5 46.15) (width 0.2) (layer "B.Cu") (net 2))
 (segment (start 107.125 46.15) (end 106.5 46.15) (width 0.2) (layer "B.Cu") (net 2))
 (segment (start 114.15 46.15) (end 116.25 48.25) (width 0.2) (layer "F.Cu") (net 1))
 (segment (start 113.825 46.15) (end 114.15 46.15) (width 0.2) (layer "F.Cu") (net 1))
 (via (at 113.825 46.15) (size 0.6) (drill 0.3) (layers "F.Cu" "B.Cu") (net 1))
 (segment (start 113.375 44.625) (end 116.25 41.75) (width 0.2) (layer "B.Cu") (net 1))
 (segment (start 113.825 46.15) (end 113.375 46.15) (width 0.2) (layer "B.Cu") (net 1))
 (segment (start 113.375 46.15) (end 113.375 44.625) (width 0.2) (layer "B.Cu") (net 1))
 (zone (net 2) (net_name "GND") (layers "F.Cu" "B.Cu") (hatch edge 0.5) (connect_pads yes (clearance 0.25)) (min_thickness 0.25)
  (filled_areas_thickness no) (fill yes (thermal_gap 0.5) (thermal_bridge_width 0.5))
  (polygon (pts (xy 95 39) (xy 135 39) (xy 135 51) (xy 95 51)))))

